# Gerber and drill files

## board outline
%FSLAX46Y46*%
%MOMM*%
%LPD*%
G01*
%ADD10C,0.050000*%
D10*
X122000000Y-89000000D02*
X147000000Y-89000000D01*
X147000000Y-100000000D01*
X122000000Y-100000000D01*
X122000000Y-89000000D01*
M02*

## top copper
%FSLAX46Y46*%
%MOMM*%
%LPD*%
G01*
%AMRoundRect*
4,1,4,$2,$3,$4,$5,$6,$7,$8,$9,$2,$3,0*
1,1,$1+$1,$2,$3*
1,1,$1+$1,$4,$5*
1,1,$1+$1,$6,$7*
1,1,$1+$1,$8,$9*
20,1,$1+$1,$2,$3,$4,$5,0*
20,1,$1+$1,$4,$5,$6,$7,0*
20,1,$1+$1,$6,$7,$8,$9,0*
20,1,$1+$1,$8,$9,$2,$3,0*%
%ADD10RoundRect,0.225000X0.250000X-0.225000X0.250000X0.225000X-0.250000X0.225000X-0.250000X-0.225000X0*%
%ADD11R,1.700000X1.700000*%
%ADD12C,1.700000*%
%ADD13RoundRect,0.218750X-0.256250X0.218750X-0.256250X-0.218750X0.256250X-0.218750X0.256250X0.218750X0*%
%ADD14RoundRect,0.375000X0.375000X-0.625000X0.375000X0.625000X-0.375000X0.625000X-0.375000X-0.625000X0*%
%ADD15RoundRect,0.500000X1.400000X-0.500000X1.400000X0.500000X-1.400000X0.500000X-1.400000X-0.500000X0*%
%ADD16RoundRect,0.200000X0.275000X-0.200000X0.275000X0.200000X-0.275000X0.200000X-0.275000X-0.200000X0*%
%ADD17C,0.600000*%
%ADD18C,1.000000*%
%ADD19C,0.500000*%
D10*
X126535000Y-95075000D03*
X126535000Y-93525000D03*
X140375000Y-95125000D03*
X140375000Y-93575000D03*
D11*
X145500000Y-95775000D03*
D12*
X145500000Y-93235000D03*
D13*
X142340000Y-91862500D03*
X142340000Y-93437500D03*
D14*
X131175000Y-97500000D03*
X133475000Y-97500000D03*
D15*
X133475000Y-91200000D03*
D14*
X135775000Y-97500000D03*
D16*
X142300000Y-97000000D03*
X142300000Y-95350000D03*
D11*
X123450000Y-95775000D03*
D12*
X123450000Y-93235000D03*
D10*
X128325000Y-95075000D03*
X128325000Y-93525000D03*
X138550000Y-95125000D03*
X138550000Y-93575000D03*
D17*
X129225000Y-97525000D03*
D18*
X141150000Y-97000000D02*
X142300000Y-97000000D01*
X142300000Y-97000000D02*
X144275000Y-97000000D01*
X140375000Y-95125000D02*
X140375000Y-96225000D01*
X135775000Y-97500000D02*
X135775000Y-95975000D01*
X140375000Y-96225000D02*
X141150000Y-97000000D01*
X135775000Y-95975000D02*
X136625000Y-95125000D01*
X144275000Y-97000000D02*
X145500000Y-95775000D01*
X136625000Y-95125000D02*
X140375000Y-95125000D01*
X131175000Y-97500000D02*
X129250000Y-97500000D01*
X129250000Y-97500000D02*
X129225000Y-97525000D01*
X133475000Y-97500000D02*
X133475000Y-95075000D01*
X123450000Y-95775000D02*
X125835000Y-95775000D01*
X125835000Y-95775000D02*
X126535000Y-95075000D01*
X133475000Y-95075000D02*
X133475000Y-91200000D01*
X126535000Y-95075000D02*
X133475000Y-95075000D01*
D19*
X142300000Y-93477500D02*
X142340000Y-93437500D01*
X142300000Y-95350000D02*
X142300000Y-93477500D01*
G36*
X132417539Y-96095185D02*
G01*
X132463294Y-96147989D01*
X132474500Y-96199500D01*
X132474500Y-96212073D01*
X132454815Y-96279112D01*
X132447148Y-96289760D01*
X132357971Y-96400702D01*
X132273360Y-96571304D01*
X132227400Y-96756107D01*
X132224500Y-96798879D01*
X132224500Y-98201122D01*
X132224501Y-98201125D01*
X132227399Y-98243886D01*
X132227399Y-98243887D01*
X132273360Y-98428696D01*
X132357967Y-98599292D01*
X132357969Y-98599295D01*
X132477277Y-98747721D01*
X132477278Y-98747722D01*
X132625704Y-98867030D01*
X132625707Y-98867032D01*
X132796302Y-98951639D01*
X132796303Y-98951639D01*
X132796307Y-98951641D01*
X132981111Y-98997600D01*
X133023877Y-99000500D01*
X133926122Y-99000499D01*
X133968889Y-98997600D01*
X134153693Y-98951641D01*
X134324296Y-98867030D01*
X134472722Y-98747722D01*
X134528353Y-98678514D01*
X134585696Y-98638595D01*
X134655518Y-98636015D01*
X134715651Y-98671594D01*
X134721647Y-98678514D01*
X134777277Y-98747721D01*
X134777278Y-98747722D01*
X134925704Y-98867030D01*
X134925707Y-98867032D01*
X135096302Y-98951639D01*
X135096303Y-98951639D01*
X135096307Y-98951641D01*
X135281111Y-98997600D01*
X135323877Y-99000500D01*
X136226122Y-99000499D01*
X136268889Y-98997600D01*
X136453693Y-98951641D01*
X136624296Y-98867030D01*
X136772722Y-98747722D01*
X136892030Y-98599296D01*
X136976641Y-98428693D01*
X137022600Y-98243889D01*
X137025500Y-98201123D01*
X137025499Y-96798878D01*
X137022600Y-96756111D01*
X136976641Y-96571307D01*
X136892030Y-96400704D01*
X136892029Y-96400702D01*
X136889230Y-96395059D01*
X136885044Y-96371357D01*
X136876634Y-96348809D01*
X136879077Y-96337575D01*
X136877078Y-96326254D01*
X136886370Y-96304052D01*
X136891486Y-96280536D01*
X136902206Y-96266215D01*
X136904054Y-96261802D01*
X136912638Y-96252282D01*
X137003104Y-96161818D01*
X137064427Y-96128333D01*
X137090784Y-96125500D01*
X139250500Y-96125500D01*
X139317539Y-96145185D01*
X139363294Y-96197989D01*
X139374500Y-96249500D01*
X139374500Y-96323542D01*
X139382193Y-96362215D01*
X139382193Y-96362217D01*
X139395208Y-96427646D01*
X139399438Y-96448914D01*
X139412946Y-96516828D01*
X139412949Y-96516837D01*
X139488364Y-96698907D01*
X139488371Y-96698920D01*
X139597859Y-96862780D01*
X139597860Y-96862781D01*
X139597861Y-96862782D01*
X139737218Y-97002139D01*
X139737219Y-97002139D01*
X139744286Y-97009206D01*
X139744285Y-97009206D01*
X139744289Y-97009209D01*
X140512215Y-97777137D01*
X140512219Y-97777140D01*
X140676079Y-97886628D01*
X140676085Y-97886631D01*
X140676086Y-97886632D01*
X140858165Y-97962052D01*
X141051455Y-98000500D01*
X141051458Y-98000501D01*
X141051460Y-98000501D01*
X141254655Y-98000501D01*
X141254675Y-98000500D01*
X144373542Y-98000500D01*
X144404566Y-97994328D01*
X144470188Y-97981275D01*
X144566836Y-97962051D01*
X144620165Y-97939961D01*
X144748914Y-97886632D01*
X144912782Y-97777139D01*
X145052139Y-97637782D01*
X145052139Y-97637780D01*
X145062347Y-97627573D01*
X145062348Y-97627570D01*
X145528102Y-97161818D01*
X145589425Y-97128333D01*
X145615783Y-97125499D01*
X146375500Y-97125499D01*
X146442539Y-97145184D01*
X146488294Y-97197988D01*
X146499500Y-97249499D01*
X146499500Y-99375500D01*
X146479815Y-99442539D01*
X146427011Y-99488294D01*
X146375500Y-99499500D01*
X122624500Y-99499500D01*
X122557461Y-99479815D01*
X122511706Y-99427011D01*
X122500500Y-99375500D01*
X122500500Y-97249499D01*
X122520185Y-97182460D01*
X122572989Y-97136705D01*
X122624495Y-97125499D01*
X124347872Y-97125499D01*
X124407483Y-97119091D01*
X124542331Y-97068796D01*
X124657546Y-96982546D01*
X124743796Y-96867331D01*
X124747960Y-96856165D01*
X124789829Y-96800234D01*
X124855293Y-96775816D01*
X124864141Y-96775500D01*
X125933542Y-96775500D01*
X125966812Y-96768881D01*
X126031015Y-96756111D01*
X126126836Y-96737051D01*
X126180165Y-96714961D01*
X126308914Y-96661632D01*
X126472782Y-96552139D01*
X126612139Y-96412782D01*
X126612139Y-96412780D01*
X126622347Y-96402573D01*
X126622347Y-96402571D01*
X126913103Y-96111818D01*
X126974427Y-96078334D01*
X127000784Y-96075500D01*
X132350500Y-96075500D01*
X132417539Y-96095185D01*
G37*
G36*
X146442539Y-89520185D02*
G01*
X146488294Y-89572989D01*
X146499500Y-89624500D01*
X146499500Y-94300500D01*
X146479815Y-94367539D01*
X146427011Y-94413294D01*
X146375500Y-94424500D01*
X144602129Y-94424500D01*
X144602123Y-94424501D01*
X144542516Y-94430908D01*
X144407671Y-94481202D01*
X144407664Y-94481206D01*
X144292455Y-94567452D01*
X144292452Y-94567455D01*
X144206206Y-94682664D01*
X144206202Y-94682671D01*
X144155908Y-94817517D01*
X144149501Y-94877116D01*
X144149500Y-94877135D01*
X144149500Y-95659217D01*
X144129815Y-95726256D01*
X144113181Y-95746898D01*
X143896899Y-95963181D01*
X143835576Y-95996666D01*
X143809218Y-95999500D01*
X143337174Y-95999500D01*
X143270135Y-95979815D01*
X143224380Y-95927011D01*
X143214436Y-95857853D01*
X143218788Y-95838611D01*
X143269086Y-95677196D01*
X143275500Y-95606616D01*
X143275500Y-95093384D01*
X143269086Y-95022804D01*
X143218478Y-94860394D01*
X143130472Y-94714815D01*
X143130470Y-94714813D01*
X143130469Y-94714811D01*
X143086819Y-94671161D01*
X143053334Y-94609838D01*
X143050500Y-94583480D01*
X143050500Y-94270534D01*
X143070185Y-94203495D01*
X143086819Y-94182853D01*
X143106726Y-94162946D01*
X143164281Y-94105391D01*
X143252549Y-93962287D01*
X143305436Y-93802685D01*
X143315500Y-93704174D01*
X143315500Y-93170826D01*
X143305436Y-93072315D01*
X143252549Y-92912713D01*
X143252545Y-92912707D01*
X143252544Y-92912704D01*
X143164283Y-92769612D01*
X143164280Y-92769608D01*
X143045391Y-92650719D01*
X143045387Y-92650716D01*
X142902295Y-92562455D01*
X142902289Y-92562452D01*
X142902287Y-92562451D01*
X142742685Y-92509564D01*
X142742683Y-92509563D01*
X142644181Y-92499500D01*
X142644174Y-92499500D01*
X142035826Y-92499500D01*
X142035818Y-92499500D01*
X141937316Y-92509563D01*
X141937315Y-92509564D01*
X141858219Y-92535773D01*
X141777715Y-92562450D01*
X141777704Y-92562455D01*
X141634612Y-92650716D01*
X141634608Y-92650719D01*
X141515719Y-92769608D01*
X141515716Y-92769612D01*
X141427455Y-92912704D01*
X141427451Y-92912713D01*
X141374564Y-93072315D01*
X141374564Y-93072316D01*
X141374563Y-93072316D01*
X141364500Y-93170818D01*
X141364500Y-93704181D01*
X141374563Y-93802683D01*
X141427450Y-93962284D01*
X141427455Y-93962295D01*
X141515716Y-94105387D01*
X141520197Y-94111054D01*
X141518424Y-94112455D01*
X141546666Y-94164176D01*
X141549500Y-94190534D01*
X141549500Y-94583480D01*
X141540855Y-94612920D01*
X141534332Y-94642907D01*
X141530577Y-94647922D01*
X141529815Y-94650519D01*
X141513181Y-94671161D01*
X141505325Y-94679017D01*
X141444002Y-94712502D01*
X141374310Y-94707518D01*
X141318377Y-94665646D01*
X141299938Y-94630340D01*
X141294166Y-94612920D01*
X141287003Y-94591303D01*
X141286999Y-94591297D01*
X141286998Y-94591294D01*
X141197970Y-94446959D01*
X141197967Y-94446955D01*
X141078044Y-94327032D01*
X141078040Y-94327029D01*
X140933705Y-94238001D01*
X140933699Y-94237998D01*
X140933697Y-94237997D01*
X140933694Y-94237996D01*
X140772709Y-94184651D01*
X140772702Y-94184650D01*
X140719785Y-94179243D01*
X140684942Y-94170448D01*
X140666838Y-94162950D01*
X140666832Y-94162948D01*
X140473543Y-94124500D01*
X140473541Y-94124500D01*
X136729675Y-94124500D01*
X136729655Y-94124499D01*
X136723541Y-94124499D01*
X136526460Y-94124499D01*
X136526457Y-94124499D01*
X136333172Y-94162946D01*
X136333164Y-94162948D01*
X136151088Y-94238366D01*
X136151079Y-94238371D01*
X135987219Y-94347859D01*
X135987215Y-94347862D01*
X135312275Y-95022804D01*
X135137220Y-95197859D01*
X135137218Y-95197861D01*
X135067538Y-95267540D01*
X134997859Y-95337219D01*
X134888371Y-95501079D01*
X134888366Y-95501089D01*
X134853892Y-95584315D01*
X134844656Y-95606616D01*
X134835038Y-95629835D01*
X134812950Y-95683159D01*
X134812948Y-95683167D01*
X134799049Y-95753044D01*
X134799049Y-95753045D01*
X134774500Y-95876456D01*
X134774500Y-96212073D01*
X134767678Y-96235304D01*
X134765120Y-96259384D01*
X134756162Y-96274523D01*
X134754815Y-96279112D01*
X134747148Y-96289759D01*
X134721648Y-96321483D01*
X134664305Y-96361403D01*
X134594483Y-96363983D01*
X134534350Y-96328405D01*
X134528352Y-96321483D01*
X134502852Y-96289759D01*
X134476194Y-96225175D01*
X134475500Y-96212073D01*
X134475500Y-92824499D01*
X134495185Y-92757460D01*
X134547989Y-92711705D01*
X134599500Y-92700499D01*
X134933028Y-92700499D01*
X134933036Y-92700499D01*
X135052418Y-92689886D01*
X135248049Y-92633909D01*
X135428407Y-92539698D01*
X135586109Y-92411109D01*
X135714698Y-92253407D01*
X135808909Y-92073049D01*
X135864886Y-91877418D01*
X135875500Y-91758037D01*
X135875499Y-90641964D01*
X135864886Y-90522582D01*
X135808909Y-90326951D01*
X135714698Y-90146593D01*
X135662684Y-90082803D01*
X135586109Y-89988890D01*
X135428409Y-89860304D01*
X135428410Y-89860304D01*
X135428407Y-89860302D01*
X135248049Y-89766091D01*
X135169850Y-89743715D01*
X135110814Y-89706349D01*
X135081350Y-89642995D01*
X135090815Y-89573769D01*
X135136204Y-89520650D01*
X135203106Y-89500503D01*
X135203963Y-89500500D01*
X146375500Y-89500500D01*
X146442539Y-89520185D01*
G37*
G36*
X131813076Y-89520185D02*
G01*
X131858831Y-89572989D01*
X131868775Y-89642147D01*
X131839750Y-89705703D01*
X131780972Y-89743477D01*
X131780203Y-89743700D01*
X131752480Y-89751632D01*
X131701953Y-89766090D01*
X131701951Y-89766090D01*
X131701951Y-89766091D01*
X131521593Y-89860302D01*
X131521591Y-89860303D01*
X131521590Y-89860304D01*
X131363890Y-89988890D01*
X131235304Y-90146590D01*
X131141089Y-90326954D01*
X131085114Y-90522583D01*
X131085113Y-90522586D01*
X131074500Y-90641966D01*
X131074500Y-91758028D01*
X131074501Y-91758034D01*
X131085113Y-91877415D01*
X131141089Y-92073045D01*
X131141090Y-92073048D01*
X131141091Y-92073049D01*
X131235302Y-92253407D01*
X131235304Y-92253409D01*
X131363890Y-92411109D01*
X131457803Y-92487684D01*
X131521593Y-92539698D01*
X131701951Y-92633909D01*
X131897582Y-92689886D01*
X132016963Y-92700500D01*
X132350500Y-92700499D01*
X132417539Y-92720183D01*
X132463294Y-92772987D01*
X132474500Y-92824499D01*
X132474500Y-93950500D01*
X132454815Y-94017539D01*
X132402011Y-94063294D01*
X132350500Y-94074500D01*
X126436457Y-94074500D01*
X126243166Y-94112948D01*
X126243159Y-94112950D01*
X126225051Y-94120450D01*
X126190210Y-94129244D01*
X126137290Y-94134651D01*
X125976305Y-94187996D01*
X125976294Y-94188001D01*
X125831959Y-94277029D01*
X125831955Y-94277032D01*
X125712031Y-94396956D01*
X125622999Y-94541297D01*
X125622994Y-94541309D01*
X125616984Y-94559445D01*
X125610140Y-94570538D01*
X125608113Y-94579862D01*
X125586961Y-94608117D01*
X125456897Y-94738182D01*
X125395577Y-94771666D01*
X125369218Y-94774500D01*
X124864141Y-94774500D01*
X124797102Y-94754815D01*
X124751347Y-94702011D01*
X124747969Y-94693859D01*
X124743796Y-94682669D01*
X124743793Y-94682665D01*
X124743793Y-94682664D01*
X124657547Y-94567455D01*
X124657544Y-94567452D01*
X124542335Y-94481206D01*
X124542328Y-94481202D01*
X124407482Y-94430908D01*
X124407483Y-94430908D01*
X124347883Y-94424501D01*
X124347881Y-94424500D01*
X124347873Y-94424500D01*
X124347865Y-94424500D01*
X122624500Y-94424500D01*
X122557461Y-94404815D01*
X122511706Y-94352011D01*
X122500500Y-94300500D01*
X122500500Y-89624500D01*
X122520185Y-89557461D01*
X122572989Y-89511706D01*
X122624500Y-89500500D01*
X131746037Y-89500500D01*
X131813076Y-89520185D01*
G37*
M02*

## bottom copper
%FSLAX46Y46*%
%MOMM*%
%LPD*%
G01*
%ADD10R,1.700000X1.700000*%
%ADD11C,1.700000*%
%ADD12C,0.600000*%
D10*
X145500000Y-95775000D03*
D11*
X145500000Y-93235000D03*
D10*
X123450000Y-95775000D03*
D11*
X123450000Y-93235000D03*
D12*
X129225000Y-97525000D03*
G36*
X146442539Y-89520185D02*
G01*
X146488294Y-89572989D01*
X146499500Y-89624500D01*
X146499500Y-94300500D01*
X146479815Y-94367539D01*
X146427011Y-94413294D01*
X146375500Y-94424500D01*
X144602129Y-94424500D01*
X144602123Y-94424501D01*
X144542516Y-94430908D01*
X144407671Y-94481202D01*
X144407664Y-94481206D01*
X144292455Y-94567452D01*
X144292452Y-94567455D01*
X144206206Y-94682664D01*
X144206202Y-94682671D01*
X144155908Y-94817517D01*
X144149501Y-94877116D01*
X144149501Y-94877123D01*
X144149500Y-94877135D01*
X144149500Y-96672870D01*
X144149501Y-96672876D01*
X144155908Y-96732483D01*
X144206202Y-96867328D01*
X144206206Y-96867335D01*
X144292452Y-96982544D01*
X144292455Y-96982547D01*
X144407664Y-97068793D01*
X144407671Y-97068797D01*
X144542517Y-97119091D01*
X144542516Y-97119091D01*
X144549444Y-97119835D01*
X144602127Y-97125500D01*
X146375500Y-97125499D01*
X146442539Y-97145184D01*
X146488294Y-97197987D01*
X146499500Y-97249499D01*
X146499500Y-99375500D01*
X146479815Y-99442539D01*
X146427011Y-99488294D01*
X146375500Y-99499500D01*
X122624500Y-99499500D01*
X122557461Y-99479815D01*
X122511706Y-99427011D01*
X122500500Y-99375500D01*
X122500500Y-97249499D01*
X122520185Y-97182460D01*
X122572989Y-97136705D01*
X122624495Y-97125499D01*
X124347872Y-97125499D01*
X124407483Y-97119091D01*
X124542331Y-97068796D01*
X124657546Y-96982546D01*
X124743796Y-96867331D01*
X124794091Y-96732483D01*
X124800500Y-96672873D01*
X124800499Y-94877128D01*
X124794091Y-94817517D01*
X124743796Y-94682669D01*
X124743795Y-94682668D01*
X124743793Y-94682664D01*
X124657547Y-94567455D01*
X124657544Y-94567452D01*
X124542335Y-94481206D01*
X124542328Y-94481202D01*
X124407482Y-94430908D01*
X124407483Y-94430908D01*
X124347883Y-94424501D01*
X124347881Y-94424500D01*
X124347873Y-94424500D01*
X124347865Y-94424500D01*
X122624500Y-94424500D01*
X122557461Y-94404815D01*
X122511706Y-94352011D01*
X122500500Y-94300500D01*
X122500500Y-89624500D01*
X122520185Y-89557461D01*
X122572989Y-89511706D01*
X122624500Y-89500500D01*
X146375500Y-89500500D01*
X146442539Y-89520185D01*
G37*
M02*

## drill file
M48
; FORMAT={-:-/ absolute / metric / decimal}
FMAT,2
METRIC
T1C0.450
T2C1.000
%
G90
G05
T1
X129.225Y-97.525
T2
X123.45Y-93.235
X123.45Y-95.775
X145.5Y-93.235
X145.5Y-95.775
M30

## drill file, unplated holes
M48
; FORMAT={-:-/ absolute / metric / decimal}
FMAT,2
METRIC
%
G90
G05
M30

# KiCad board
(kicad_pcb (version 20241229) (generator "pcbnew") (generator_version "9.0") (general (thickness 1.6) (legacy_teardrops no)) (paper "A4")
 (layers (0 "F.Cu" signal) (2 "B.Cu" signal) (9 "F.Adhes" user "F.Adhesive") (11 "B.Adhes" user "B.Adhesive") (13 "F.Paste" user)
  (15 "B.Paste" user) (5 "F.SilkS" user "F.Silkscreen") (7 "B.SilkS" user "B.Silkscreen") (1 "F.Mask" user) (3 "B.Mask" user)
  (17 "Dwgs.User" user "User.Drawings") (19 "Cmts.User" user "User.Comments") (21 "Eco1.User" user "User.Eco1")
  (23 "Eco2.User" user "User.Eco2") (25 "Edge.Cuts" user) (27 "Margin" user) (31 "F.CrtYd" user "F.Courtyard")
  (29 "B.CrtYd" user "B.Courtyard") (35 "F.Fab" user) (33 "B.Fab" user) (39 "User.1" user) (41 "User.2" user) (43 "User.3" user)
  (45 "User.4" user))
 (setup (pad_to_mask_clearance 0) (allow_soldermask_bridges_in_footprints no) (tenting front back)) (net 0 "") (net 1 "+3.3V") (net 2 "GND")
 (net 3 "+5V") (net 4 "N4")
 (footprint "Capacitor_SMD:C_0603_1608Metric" (layer "F.Cu") (at 126.535 94.3 90)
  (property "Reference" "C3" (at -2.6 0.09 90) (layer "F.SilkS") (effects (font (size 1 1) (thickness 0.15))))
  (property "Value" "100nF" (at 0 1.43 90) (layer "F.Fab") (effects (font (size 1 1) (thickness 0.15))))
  (pad "1" smd roundrect (at -0.775 0 90) (size 0.9 0.95) (layers "F.Cu" "F.Mask" "F.Paste") (roundrect_rratio 0.25) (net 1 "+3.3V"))
  (pad "2" smd roundrect (at 0.775 0 90) (size 0.9 0.95) (layers "F.Cu" "F.Mask" "F.Paste") (roundrect_rratio 0.25) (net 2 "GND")))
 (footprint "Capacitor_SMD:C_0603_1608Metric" (layer "F.Cu") (at 140.375 94.35 90)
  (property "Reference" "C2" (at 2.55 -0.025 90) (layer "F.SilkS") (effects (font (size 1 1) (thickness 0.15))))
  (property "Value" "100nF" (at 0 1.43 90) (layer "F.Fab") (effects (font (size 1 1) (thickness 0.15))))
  (pad "1" smd roundrect (at -0.775 0 90) (size 0.9 0.95) (layers "F.Cu" "F.Mask" "F.Paste") (roundrect_rratio 0.25) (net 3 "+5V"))
  (pad "2" smd roundrect (at 0.775 0 90) (size 0.9 0.95) (layers "F.Cu" "F.Mask" "F.Paste") (roundrect_rratio 0.25) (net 2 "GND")))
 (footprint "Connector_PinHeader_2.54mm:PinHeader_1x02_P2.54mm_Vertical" (layer "F.Cu") (at 145.5 95.775 180)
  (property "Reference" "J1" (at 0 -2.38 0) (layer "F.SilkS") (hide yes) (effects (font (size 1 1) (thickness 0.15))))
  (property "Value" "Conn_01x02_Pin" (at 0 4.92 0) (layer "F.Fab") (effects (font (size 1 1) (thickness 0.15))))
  (pad "1" thru_hole rect (at 0 0 180) (size 1.7 1.7) (drill 1) (layers "*.Cu" "*.Mask") (remove_unused_layers no) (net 3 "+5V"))
  (pad "2" thru_hole circle (at 0 2.54 180) (size 1.7 1.7) (drill 1) (layers "*.Cu" "*.Mask") (remove_unused_layers no) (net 2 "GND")))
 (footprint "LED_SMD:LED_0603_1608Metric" (layer "F.Cu") (at 142.34 92.65 -90)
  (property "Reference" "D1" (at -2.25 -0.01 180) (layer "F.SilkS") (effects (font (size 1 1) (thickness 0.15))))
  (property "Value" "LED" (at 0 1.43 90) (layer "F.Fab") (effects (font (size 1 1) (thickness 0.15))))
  (pad "1" smd roundrect (at -0.7875 0 270) (size 0.875 0.95) (layers "F.Cu" "F.Mask" "F.Paste") (roundrect_rratio 0.25) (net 2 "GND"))
  (pad "2" smd roundrect (at 0.7875 0 270) (size 0.875 0.95) (layers "F.Cu" "F.Mask" "F.Paste") (roundrect_rratio 0.25) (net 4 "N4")))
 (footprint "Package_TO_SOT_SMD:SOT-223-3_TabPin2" (layer "F.Cu") (at 133.475 94.35 90)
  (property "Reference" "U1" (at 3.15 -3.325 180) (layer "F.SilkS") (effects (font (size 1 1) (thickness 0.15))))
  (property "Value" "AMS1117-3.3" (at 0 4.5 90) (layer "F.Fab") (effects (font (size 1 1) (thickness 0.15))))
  (pad "1" smd roundrect (at -3.15 -2.3 90) (size 2 1.5) (layers "F.Cu" "F.Mask" "F.Paste") (roundrect_rratio 0.25) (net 2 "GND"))
  (pad "2" smd roundrect (at -3.15 0 90) (size 2 1.5) (layers "F.Cu" "F.Mask" "F.Paste") (roundrect_rratio 0.25) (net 1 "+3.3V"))
  (pad "2" smd roundrect (at 3.15 0 90) (size 2 3.8) (layers "F.Cu" "F.Mask" "F.Paste") (roundrect_rratio 0.25) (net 1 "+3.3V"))
  (pad "3" smd roundrect (at -3.15 2.3 90) (size 2 1.5) (layers "F.Cu" "F.Mask" "F.Paste") (roundrect_rratio 0.25) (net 3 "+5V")))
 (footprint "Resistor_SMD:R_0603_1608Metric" (layer "F.Cu") (at 142.3 96.175 90)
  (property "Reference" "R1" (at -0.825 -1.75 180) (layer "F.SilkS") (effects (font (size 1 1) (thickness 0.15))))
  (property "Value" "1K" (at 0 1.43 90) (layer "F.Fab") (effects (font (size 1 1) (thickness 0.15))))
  (pad "1" smd roundrect (at -0.825 0 90) (size 0.8 0.95) (layers "F.Cu" "F.Mask" "F.Paste") (roundrect_rratio 0.25) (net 3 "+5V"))
  (pad "2" smd roundrect (at 0.825 0 90) (size 0.8 0.95) (layers "F.Cu" "F.Mask" "F.Paste") (roundrect_rratio 0.25) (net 4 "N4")))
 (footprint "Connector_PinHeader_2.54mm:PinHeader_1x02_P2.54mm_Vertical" (layer "F.Cu") (at 123.45 95.775 180)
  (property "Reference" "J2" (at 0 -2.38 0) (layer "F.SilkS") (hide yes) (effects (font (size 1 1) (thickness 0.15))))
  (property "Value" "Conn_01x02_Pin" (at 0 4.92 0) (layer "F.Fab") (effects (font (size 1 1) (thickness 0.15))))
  (pad "1" thru_hole rect (at 0 0 180) (size 1.7 1.7) (drill 1) (layers "*.Cu" "*.Mask") (remove_unused_layers no) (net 1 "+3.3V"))
  (pad "2" thru_hole circle (at 0 2.54 180) (size 1.7 1.7) (drill 1) (layers "*.Cu" "*.Mask") (remove_unused_layers no) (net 2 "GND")))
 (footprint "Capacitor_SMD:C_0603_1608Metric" (layer "F.Cu") (at 128.325 94.3 90)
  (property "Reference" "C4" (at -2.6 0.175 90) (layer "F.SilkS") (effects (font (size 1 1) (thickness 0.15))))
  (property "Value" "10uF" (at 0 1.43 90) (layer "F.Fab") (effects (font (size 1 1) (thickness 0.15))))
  (pad "1" smd roundrect (at -0.775 0 90) (size 0.9 0.95) (layers "F.Cu" "F.Mask" "F.Paste") (roundrect_rratio 0.25) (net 1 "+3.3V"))
  (pad "2" smd roundrect (at 0.775 0 90) (size 0.9 0.95) (layers "F.Cu" "F.Mask" "F.Paste") (roundrect_rratio 0.25) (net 2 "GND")))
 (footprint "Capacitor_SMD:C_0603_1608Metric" (layer "F.Cu") (at 138.55 94.35 90)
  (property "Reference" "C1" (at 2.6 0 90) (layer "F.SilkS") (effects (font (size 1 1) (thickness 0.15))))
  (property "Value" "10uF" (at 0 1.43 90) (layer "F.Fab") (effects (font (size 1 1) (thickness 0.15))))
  (pad "1" smd roundrect (at -0.775 0 90) (size 0.9 0.95) (layers "F.Cu" "F.Mask" "F.Paste") (roundrect_rratio 0.25) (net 3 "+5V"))
  (pad "2" smd roundrect (at 0.775 0 90) (size 0.9 0.95) (layers "F.Cu" "F.Mask" "F.Paste") (roundrect_rratio 0.25) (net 2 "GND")))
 (gr_rect (start 122 89) (end 147 100) (stroke (width 0.05) (type default)) (fill no) (layer "Edge.Cuts"))
 (segment (start 141.15 97) (end 142.3 97) (width 1) (layer "F.Cu") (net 3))
 (segment (start 142.3 97) (end 144.275 97) (width 1) (layer "F.Cu") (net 3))
 (segment (start 140.375 95.125) (end 140.375 96.225) (width 1) (layer "F.Cu") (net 3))
 (segment (start 135.775 97.5) (end 135.775 95.975) (width 1) (layer "F.Cu") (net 3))
 (segment (start 140.375 96.225) (end 141.15 97) (width 1) (layer "F.Cu") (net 3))
 (segment (start 135.775 95.975) (end 136.625 95.125) (width 1) (layer "F.Cu") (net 3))
 (segment (start 144.275 97) (end 145.5 95.775) (width 1) (layer "F.Cu") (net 3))
 (segment (start 136.625 95.125) (end 140.375 95.125) (width 1) (layer "F.Cu") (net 3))
 (segment (start 131.175 97.5) (end 129.25 97.5) (width 1) (layer "F.Cu") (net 2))
 (segment (start 129.25 97.5) (end 129.225 97.525) (width 1) (layer "F.Cu") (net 2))
 (via (at 129.225 97.525) (size 0.6) (drill 0.45) (layers "F.Cu" "B.Cu") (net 2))
 (segment (start 133.475 97.5) (end 133.475 95.075) (width 1) (layer "F.Cu") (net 1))
 (segment (start 123.45 95.775) (end 125.835 95.775) (width 1) (layer "F.Cu") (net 1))
 (segment (start 125.835 95.775) (end 126.535 95.075) (width 1) (layer "F.Cu") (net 1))
 (segment (start 133.475 95.075) (end 133.475 91.2) (width 1) (layer "F.Cu") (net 1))
 (segment (start 126.535 95.075) (end 133.475 95.075) (width 1) (layer "F.Cu") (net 1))
 (segment (start 142.3 93.4775) (end 142.34 93.4375) (width 0.5) (layer "F.Cu") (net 4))
 (segment (start 142.3 95.35) (end 142.3 93.4775) (width 0.5) (layer "F.Cu") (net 4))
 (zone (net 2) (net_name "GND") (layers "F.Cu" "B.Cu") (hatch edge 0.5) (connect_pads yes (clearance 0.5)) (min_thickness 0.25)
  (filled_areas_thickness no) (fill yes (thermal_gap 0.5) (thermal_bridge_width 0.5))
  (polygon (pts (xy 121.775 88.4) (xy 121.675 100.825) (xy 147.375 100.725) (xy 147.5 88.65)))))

